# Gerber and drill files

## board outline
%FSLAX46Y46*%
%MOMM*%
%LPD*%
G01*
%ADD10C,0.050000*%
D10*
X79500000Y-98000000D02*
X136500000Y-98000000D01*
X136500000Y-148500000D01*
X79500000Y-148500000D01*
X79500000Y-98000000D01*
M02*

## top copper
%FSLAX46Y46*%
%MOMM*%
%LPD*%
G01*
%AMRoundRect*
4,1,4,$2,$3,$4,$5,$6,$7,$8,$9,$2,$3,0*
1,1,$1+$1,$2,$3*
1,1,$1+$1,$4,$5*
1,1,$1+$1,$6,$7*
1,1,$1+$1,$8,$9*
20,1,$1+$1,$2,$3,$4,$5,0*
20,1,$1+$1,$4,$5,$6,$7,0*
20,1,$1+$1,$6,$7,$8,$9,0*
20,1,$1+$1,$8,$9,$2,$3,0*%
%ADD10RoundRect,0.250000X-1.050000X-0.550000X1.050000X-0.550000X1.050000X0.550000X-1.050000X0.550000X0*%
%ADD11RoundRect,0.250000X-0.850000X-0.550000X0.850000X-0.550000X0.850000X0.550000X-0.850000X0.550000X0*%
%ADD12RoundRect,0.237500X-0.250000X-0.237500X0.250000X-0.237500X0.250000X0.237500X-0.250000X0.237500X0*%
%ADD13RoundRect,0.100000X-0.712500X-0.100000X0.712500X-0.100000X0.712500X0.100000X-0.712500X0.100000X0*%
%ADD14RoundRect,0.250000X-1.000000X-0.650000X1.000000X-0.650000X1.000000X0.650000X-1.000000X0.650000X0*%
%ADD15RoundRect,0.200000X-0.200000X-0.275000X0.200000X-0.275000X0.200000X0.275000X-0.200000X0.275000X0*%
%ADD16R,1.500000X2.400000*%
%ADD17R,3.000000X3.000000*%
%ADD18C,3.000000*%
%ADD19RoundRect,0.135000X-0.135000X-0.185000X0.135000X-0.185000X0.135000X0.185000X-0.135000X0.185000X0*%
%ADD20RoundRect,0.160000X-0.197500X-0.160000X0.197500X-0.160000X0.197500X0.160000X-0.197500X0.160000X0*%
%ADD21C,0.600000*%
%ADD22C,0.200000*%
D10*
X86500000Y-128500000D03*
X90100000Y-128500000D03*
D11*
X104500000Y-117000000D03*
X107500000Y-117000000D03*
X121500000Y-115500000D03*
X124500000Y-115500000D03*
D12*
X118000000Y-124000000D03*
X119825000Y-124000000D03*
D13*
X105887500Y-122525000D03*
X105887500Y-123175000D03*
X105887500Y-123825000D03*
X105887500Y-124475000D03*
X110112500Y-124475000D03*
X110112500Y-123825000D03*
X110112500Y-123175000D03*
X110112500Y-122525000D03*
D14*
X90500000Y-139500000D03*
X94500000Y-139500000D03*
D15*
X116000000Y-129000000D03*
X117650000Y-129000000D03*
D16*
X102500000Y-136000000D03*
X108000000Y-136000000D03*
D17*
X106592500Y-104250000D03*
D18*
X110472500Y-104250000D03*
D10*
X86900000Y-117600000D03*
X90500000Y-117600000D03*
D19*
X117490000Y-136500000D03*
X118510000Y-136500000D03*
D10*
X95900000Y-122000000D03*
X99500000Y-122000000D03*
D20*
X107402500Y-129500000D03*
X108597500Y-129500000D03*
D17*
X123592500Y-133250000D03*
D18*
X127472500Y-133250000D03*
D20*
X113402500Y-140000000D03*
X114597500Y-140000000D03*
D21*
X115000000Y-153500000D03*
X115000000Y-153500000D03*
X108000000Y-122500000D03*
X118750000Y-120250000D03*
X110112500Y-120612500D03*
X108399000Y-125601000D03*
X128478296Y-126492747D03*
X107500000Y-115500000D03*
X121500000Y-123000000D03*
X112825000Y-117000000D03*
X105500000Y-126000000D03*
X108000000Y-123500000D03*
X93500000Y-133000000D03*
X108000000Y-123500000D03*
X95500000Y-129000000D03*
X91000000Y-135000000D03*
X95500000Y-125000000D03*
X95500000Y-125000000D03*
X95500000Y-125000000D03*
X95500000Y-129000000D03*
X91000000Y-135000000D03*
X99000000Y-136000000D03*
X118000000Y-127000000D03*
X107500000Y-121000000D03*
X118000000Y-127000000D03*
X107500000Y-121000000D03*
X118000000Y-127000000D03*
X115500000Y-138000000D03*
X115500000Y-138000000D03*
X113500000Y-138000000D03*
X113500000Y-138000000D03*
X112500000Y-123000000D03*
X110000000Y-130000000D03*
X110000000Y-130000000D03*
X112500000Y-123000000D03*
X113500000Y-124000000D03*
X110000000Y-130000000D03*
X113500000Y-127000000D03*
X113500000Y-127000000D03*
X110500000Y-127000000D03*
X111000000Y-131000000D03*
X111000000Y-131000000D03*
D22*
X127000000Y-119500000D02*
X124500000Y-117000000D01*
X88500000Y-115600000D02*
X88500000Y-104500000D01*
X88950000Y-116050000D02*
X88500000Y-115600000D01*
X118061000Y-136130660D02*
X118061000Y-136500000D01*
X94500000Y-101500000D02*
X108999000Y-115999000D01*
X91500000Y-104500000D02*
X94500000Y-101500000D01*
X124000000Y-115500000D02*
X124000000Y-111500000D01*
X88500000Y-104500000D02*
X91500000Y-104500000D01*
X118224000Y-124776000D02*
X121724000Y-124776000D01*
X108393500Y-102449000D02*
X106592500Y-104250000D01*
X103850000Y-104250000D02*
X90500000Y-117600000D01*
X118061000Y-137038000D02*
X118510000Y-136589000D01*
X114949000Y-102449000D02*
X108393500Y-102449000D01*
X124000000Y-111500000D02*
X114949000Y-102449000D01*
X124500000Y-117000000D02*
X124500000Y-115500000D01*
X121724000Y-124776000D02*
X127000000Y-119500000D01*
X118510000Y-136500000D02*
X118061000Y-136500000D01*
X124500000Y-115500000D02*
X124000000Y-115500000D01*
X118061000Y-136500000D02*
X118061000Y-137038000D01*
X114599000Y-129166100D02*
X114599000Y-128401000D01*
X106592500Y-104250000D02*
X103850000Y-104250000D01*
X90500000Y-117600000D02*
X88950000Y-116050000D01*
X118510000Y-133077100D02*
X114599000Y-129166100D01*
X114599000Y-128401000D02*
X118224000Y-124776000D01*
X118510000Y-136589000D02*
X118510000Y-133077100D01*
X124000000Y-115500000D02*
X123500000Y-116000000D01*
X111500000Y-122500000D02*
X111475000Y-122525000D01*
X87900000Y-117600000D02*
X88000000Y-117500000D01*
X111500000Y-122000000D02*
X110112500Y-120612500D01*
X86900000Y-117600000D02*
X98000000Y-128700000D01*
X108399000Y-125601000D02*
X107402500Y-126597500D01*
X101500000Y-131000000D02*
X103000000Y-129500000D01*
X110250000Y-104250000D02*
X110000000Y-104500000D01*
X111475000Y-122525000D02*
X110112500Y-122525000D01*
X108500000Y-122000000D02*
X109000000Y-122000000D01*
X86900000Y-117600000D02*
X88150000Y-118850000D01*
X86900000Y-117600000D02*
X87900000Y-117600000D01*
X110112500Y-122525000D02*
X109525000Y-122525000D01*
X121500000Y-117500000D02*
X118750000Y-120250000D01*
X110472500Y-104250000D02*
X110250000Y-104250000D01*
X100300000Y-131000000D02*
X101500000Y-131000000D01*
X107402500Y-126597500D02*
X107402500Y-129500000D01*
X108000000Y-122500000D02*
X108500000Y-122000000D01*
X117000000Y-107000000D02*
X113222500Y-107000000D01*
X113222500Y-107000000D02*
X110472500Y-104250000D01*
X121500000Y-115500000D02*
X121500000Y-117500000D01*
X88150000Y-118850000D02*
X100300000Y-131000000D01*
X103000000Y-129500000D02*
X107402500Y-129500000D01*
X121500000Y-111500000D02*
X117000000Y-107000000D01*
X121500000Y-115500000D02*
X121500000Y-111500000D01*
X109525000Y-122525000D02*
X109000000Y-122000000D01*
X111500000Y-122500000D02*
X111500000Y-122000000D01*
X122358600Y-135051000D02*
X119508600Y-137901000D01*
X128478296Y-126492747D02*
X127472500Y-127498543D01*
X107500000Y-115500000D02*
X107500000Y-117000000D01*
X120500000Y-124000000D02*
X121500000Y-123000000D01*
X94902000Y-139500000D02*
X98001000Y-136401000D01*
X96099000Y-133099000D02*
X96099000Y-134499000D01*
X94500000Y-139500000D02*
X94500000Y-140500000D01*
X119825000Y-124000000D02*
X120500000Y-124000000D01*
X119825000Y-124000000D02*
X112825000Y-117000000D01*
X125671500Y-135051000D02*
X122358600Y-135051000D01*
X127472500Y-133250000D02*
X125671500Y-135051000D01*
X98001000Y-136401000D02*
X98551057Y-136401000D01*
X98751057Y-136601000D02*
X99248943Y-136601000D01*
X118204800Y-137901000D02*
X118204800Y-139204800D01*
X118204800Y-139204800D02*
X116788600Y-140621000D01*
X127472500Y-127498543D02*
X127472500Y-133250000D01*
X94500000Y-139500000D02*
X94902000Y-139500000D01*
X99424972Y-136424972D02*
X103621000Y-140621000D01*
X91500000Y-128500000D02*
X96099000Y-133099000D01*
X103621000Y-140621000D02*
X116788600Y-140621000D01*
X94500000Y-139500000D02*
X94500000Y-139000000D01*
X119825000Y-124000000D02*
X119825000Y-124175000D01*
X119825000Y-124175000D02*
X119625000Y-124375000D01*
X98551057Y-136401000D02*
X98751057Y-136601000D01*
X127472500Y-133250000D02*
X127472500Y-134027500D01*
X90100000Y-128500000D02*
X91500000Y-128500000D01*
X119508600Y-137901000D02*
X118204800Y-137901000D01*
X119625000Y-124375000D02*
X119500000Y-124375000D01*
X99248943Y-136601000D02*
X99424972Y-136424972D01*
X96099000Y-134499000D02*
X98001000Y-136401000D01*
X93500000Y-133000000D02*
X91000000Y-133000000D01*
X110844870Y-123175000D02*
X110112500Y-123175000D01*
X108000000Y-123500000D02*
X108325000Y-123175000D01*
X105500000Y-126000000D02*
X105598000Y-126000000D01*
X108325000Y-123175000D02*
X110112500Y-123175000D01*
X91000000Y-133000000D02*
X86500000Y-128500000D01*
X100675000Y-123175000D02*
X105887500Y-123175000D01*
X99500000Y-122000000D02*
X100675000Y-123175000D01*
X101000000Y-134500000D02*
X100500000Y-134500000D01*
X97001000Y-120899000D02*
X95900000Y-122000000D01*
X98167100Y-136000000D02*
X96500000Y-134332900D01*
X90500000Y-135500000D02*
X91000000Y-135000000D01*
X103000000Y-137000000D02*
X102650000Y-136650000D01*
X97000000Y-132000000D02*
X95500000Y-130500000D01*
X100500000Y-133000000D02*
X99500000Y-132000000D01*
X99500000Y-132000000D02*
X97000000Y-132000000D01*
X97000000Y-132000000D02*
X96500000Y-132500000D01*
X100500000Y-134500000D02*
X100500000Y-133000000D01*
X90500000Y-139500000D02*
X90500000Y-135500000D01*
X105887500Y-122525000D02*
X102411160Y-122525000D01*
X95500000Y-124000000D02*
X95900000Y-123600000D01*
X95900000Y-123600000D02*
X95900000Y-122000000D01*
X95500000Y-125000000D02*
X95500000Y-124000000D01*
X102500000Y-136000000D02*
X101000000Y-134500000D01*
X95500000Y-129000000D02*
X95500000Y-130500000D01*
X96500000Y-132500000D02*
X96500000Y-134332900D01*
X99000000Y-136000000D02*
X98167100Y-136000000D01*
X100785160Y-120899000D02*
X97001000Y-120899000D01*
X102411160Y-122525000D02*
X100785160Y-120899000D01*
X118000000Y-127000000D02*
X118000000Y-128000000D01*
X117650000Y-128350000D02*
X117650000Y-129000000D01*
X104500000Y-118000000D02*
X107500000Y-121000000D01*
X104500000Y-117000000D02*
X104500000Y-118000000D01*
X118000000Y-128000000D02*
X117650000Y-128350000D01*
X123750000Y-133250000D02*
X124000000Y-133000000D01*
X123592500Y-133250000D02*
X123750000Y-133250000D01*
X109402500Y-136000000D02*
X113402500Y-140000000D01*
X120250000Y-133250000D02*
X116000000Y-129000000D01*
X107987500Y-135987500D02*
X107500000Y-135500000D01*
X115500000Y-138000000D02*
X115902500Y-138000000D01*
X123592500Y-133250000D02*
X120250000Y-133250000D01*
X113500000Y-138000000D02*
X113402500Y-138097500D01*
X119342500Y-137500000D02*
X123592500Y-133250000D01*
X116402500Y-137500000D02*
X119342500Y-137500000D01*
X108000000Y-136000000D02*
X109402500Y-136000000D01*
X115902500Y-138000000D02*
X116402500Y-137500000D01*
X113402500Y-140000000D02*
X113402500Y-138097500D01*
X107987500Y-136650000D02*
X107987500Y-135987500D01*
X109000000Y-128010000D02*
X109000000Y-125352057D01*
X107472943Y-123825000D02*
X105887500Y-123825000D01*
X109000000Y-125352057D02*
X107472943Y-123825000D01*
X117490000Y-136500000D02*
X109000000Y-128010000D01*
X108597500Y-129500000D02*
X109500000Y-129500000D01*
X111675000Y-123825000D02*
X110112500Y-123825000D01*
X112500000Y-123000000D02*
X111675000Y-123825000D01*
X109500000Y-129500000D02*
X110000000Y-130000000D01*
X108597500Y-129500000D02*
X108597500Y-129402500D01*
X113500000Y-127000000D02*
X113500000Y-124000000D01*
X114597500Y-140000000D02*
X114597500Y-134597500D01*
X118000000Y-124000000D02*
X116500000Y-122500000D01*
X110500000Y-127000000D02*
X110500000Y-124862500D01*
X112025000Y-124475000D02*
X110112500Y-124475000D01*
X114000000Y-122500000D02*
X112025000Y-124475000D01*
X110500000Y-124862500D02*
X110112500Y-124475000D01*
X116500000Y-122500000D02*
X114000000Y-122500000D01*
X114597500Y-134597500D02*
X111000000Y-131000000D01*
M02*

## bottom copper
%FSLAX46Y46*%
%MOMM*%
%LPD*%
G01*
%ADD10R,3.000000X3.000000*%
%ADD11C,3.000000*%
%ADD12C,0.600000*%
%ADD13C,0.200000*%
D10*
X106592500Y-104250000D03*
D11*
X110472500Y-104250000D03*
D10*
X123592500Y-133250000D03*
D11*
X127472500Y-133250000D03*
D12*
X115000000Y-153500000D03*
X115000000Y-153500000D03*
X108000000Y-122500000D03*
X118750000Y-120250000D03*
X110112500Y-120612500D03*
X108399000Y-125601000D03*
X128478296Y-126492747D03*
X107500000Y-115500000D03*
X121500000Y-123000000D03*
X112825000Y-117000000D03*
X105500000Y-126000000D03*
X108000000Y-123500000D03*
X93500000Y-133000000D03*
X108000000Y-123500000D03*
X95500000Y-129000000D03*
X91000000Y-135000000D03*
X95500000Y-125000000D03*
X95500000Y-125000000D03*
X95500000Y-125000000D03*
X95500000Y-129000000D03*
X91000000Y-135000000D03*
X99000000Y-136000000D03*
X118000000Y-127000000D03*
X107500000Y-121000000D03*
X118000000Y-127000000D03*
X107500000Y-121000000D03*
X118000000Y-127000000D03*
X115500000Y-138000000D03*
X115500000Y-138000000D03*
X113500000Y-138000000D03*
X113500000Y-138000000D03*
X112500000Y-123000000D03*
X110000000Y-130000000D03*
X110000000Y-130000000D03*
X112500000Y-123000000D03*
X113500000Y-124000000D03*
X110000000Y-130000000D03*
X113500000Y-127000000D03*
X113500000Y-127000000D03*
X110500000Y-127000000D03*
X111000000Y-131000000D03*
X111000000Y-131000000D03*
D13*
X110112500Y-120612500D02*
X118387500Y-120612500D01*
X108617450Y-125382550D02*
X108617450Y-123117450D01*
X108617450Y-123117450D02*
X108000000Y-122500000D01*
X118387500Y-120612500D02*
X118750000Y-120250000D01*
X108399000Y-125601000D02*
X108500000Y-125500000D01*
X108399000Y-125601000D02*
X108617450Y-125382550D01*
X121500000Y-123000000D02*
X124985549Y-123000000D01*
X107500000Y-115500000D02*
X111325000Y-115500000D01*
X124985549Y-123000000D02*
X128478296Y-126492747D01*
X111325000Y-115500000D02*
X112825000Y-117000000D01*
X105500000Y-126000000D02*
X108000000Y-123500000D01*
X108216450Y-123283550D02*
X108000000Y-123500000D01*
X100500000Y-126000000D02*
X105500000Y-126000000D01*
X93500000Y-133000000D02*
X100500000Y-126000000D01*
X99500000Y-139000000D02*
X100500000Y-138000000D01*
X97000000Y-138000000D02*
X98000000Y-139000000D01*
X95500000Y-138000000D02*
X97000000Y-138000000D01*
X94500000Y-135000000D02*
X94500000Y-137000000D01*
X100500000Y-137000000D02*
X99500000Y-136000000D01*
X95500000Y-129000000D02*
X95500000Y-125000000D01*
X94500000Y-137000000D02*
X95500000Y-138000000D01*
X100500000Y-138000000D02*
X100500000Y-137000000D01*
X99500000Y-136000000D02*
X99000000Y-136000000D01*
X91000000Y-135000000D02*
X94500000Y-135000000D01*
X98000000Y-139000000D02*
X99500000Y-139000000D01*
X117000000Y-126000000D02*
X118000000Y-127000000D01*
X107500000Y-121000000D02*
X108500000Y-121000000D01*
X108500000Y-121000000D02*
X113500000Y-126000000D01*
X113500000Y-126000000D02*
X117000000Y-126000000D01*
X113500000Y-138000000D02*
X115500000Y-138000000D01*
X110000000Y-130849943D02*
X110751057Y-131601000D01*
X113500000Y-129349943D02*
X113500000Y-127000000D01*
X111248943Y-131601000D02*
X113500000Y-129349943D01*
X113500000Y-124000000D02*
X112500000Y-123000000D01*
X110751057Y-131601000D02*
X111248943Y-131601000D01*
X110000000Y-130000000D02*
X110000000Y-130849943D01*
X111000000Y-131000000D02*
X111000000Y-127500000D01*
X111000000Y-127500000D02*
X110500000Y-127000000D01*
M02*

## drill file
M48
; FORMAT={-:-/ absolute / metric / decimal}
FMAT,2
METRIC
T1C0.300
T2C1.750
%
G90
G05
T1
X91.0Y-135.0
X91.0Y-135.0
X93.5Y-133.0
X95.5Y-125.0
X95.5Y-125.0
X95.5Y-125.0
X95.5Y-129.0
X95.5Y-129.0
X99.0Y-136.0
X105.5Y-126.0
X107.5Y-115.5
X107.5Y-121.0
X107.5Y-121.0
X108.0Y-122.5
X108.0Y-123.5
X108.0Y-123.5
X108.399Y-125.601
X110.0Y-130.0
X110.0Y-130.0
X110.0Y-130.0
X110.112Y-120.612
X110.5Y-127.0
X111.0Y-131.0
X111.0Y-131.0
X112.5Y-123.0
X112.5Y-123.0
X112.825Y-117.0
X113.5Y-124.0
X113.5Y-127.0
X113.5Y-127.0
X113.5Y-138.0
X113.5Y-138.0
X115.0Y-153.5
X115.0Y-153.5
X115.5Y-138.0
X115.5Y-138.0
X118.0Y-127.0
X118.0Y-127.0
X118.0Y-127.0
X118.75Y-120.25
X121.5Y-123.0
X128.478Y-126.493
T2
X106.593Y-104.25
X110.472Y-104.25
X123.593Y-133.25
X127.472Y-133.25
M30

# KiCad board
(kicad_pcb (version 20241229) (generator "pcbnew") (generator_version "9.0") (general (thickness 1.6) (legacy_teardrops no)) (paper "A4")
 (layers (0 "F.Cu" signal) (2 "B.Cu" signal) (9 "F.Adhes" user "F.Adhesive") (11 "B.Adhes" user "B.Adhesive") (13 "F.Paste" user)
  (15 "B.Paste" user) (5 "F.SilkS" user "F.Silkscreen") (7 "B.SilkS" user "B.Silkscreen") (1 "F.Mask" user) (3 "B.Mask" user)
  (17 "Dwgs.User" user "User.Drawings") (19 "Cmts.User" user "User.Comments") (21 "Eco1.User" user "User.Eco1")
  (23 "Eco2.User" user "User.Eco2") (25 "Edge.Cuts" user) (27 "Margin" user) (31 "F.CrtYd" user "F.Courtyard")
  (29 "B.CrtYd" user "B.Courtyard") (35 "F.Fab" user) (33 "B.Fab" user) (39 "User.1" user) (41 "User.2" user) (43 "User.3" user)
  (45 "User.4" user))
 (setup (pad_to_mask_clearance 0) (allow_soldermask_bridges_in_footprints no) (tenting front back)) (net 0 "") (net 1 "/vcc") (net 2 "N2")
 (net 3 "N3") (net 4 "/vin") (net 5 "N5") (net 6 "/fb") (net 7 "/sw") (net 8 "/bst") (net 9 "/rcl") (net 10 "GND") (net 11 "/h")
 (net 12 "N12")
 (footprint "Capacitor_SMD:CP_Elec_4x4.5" (layer "F.Cu") (at 88.3 128.5)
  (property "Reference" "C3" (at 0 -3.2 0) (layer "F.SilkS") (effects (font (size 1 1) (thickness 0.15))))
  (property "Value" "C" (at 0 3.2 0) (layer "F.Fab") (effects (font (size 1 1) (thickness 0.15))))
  (pad "1" smd roundrect (at -1.8 0) (size 2.6 1.6) (layers "F.Cu" "F.Mask" "F.Paste") (roundrect_rratio 0.15625) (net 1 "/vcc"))
  (pad "2" smd roundrect (at 1.8 0) (size 2.6 1.6) (layers "F.Cu" "F.Mask" "F.Paste") (roundrect_rratio 0.15625) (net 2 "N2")))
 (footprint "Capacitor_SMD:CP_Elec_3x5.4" (layer "F.Cu") (at 106 117)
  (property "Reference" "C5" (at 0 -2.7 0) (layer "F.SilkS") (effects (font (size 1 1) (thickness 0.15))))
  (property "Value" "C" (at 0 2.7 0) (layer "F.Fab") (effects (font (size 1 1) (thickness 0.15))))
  (pad "1" smd roundrect (at -1.5 0) (size 2.2 1.6) (layers "F.Cu" "F.Mask" "F.Paste") (roundrect_rratio 0.15625) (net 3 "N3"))
  (pad "2" smd roundrect (at 1.5 0) (size 2.2 1.6) (layers "F.Cu" "F.Mask" "F.Paste") (roundrect_rratio 0.15625) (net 2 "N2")))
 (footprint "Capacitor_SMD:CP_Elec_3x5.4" (layer "F.Cu") (at 123 115.5)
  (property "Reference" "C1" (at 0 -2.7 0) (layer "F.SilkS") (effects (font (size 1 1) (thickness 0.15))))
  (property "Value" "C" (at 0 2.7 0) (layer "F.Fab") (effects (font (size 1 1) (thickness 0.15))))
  (pad "1" smd roundrect (at -1.5 0) (size 2.2 1.6) (layers "F.Cu" "F.Mask" "F.Paste") (roundrect_rratio 0.15625) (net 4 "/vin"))
  (pad "2" smd roundrect (at 1.5 0) (size 2.2 1.6) (layers "F.Cu" "F.Mask" "F.Paste") (roundrect_rratio 0.15625) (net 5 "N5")))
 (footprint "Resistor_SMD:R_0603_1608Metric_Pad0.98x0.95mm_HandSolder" (layer "F.Cu") (at 118.9125 124)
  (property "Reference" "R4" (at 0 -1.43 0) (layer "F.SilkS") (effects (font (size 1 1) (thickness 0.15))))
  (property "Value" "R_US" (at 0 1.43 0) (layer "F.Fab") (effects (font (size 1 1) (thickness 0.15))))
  (pad "1" smd roundrect (at -0.9125 0) (size 0.975 0.95) (layers "F.Cu" "F.Mask" "F.Paste") (roundrect_rratio 0.25) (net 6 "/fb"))
  (pad "2" smd roundrect (at 0.9125 0) (size 0.975 0.95) (layers "F.Cu" "F.Mask" "F.Paste") (roundrect_rratio 0.25) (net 2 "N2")))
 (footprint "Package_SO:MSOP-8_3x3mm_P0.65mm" (layer "F.Cu") (at 108 123.5)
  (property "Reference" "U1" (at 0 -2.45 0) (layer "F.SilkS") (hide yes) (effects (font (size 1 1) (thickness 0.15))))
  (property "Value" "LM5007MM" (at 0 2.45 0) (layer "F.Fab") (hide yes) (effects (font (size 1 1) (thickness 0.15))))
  (pad "1" smd roundrect (at -2.1125 -0.975) (size 1.625 0.4) (layers "F.Cu" "F.Mask" "F.Paste") (roundrect_rratio 0.25) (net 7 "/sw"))
  (pad "2" smd roundrect (at -2.1125 -0.325) (size 1.625 0.4) (layers "F.Cu" "F.Mask" "F.Paste") (roundrect_rratio 0.25) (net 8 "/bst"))
  (pad "3" smd roundrect (at -2.1125 0.325) (size 1.625 0.4) (layers "F.Cu" "F.Mask" "F.Paste") (roundrect_rratio 0.25) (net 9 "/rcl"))
  (pad "4" smd roundrect (at -2.1125 0.975) (size 1.625 0.4) (layers "F.Cu" "F.Mask" "F.Paste") (roundrect_rratio 0.25) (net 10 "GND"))
  (pad "5" smd roundrect (at 2.1125 0.975) (size 1.625 0.4) (layers "F.Cu" "F.Mask" "F.Paste") (roundrect_rratio 0.25) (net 6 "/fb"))
  (pad "6" smd roundrect (at 2.1125 0.325) (size 1.625 0.4) (layers "F.Cu" "F.Mask" "F.Paste") (roundrect_rratio 0.25) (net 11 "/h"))
  (pad "7" smd roundrect (at 2.1125 -0.325) (size 1.625 0.4) (layers "F.Cu" "F.Mask" "F.Paste") (roundrect_rratio 0.25) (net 1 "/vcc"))
  (pad "8" smd roundrect (at 2.1125 -0.975) (size 1.625 0.4) (layers "F.Cu" "F.Mask" "F.Paste") (roundrect_rratio 0.25) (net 4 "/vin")))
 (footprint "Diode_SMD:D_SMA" (layer "F.Cu") (at 92.5 139.5)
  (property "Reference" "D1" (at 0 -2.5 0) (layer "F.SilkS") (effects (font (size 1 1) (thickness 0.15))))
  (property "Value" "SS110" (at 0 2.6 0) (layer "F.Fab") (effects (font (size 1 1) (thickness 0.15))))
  (pad "1" smd roundrect (at -2 0) (size 2.5 1.8) (layers "F.Cu" "F.Mask" "F.Paste") (roundrect_rratio 0.1388888889) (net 7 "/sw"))
  (pad "2" smd roundrect (at 2 0) (size 2.5 1.8) (layers "F.Cu" "F.Mask" "F.Paste") (roundrect_rratio 0.1388888889) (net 2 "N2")))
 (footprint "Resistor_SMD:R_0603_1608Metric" (layer "F.Cu") (at 116.825 129)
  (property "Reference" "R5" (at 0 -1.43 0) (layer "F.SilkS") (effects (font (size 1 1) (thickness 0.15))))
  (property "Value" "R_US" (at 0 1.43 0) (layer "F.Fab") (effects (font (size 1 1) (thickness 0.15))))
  (pad "1" smd roundrect (at -0.825 0) (size 0.8 0.95) (layers "F.Cu" "F.Mask" "F.Paste") (roundrect_rratio 0.25) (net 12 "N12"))
  (pad "2" smd roundrect (at 0.825 0) (size 0.8 0.95) (layers "F.Cu" "F.Mask" "F.Paste") (roundrect_rratio 0.25) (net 3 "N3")))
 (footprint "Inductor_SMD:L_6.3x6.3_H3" (layer "F.Cu") (at 105.25 136)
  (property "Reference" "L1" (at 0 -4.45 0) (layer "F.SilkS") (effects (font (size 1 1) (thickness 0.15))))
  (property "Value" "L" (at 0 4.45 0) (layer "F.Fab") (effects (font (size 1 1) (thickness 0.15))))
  (pad "1" smd rect (at -2.75 0) (size 1.5 2.4) (layers "F.Cu" "F.Mask" "F.Paste") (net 7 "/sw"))
  (pad "2" smd rect (at 2.75 0) (size 1.5 2.4) (layers "F.Cu" "F.Mask" "F.Paste") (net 12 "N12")))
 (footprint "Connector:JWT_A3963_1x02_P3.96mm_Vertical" (layer "F.Cu") (at 106.5925 104.25)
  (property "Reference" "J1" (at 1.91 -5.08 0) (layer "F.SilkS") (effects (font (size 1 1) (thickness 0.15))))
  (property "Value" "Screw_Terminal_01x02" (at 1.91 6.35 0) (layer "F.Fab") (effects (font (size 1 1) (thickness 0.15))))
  (pad "1" thru_hole rect (at 0 0) (size 3 3) (drill 1.75) (layers "*.Cu" "*.Mask") (remove_unused_layers no) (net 5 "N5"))
  (pad "2" thru_hole circle (at 3.88 0) (size 3 3) (drill 1.75) (layers "*.Cu" "*.Mask") (remove_unused_layers no) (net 4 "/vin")))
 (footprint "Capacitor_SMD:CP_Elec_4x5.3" (layer "F.Cu") (at 88.7 117.6)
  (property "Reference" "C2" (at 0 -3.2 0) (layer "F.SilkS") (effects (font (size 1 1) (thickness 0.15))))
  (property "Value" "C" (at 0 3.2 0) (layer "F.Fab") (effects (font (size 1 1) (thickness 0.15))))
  (pad "1" smd roundrect (at -1.8 0) (size 2.6 1.6) (layers "F.Cu" "F.Mask" "F.Paste") (roundrect_rratio 0.15625) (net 4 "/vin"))
  (pad "2" smd roundrect (at 1.8 0) (size 2.6 1.6) (layers "F.Cu" "F.Mask" "F.Paste") (roundrect_rratio 0.15625) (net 5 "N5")))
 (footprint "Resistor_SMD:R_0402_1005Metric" (layer "F.Cu") (at 118 136.5)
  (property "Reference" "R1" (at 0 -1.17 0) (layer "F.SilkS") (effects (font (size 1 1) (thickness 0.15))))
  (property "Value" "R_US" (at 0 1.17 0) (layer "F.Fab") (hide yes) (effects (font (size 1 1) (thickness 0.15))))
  (pad "1" smd roundrect (at -0.51 0) (size 0.54 0.64) (layers "F.Cu" "F.Mask" "F.Paste") (roundrect_rratio 0.25) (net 9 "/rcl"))
  (pad "2" smd roundrect (at 0.51 0) (size 0.54 0.64) (layers "F.Cu" "F.Mask" "F.Paste") (roundrect_rratio 0.25) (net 5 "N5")))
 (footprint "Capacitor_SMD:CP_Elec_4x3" (layer "F.Cu") (at 97.7 122)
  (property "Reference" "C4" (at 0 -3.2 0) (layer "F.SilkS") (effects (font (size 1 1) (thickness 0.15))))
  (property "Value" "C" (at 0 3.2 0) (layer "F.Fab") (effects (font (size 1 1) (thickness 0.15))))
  (pad "1" smd roundrect (at -1.8 0) (size 2.6 1.6) (layers "F.Cu" "F.Mask" "F.Paste") (roundrect_rratio 0.15625) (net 7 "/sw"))
  (pad "2" smd roundrect (at 1.8 0) (size 2.6 1.6) (layers "F.Cu" "F.Mask" "F.Paste") (roundrect_rratio 0.15625) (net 8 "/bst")))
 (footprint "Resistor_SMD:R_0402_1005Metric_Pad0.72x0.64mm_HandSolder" (layer "F.Cu") (at 108 129.5)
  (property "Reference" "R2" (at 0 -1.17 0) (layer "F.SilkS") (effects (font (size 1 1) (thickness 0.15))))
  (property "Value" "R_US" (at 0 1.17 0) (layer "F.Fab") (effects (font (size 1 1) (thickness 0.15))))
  (pad "1" smd roundrect (at -0.5975 0) (size 0.715 0.64) (layers "F.Cu" "F.Mask" "F.Paste") (roundrect_rratio 0.25) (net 4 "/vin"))
  (pad "2" smd roundrect (at 0.5975 0) (size 0.715 0.64) (layers "F.Cu" "F.Mask" "F.Paste") (roundrect_rratio 0.25) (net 11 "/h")))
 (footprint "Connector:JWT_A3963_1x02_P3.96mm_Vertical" (layer "F.Cu") (at 123.5925 133.25)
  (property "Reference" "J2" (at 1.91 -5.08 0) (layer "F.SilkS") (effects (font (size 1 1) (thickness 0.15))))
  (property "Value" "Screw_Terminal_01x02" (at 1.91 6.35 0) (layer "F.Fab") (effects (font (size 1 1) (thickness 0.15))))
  (pad "1" thru_hole rect (at 0 0) (size 3 3) (drill 1.75) (layers "*.Cu" "*.Mask") (remove_unused_layers no) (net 12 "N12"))
  (pad "2" thru_hole circle (at 3.88 0) (size 3 3) (drill 1.75) (layers "*.Cu" "*.Mask") (remove_unused_layers no) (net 2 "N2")))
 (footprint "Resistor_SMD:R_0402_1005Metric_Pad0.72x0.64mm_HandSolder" (layer "F.Cu") (at 114 140)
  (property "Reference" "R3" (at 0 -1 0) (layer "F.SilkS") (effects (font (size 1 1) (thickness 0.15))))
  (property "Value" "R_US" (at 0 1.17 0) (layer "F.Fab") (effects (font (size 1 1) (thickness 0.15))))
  (pad "1" smd roundrect (at -0.5975 0) (size 0.715 0.64) (layers "F.Cu" "F.Mask" "F.Paste") (roundrect_rratio 0.25) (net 12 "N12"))
  (pad "2" smd roundrect (at 0.5975 0) (size 0.715 0.64) (layers "F.Cu" "F.Mask" "F.Paste") (roundrect_rratio 0.25) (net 6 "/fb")))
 (gr_rect (start 79.5 98) (end 136.5 148.5) (stroke (width 0.05) (type default)) (fill no) (layer "Edge.Cuts"))
 (via (at 115 153.5) (size 0.6) (drill 0.3) (layers "F.Cu" "B.Cu") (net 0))
 (via (at 115 153.5) (size 0.6) (drill 0.3) (layers "F.Cu" "B.Cu") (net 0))
 (segment (start 127 119.5) (end 124.5 117) (width 0.2) (layer "F.Cu") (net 5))
 (segment (start 88.5 115.6) (end 88.5 104.5) (width 0.2) (layer "F.Cu") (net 5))
 (segment (start 88.95 116.05) (end 88.5 115.6) (width 0.2) (layer "F.Cu") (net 5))
 (segment (start 118.061 136.13066) (end 118.061 136.5) (width 0.2) (layer "F.Cu") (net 5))
 (segment (start 94.5 101.5) (end 108.999 115.999) (width 0.2) (layer "F.Cu") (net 5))
 (segment (start 91.5 104.5) (end 94.5 101.5) (width 0.2) (layer "F.Cu") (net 5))
 (segment (start 124 115.5) (end 124 111.5) (width 0.2) (layer "F.Cu") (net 5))
 (segment (start 88.5 104.5) (end 91.5 104.5) (width 0.2) (layer "F.Cu") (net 5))
 (segment (start 118.224 124.776) (end 121.724 124.776) (width 0.2) (layer "F.Cu") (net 5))
 (segment (start 108.3935 102.449) (end 106.5925 104.25) (width 0.2) (layer "F.Cu") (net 5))
 (segment (start 103.85 104.25) (end 90.5 117.6) (width 0.2) (layer "F.Cu") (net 5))
 (segment (start 118.061 137.038) (end 118.51 136.589) (width 0.2) (layer "F.Cu") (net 5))
 (segment (start 114.949 102.449) (end 108.3935 102.449) (width 0.2) (layer "F.Cu") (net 5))
 (segment (start 124 111.5) (end 114.949 102.449) (width 0.2) (layer "F.Cu") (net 5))
 (segment (start 124.5 117) (end 124.5 115.5) (width 0.2) (layer "F.Cu") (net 5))
 (segment (start 121.724 124.776) (end 127 119.5) (width 0.2) (layer "F.Cu") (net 5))
 (segment (start 118.51 136.5) (end 118.061 136.5) (width 0.2) (layer "F.Cu") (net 5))
 (segment (start 124.5 115.5) (end 124 115.5) (width 0.2) (layer "F.Cu") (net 5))
 (segment (start 118.061 136.5) (end 118.061 137.038) (width 0.2) (layer "F.Cu") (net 5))
 (segment (start 114.599 129.1661) (end 114.599 128.401) (width 0.2) (layer "F.Cu") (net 5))
 (segment (start 106.5925 104.25) (end 103.85 104.25) (width 0.2) (layer "F.Cu") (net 5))
 (segment (start 90.5 117.6) (end 88.95 116.05) (width 0.2) (layer "F.Cu") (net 5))
 (segment (start 118.51 133.0771) (end 114.599 129.1661) (width 0.2) (layer "F.Cu") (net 5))
 (segment (start 114.599 128.401) (end 118.224 124.776) (width 0.2) (layer "F.Cu") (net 5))
 (segment (start 118.51 136.589) (end 118.51 133.0771) (width 0.2) (layer "F.Cu") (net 5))
 (segment (start 124 115.5) (end 123.5 116) (width 0.2) (layer "F.Cu") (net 5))
 (segment (start 111.5 122.5) (end 111.475 122.525) (width 0.2) (layer "F.Cu") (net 4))
 (segment (start 87.9 117.6) (end 88 117.5) (width 0.2) (layer "F.Cu") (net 4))
 (segment (start 111.5 122) (end 110.1125 120.6125) (width 0.2) (layer "F.Cu") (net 4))
 (segment (start 86.9 117.6) (end 98 128.7) (width 0.2) (layer "F.Cu") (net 4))
 (segment (start 108.399 125.601) (end 107.4025 126.5975) (width 0.2) (layer "F.Cu") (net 4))
 (segment (start 101.5 131) (end 103 129.5) (width 0.2) (layer "F.Cu") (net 4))
 (segment (start 110.25 104.25) (end 110 104.5) (width 0.2) (layer "F.Cu") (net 4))
 (segment (start 111.475 122.525) (end 110.1125 122.525) (width 0.2) (layer "F.Cu") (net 4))
 (segment (start 108.5 122) (end 109 122) (width 0.2) (layer "F.Cu") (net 4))
 (segment (start 86.9 117.6) (end 88.15 118.85) (width 0.2) (layer "F.Cu") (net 4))
 (segment (start 86.9 117.6) (end 87.9 117.6) (width 0.2) (layer "F.Cu") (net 4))
 (segment (start 110.1125 122.525) (end 109.525 122.525) (width 0.2) (layer "F.Cu") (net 4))
 (segment (start 121.5 117.5) (end 118.75 120.25) (width 0.2) (layer "F.Cu") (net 4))
 (segment (start 110.4725 104.25) (end 110.25 104.25) (width 0.2) (layer "F.Cu") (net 4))
 (segment (start 100.3 131) (end 101.5 131) (width 0.2) (layer "F.Cu") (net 4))
 (segment (start 107.4025 126.5975) (end 107.4025 129.5) (width 0.2) (layer "F.Cu") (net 4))
 (segment (start 108 122.5) (end 108.5 122) (width 0.2) (layer "F.Cu") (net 4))
 (segment (start 117 107) (end 113.2225 107) (width 0.2) (layer "F.Cu") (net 4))
 (segment (start 113.2225 107) (end 110.4725 104.25) (width 0.2) (layer "F.Cu") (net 4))
 (segment (start 121.5 115.5) (end 121.5 117.5) (width 0.2) (layer "F.Cu") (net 4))
 (segment (start 88.15 118.85) (end 100.3 131) (width 0.2) (layer "F.Cu") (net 4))
 (segment (start 103 129.5) (end 107.4025 129.5) (width 0.2) (layer "F.Cu") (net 4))
 (segment (start 121.5 111.5) (end 117 107) (width 0.2) (layer "F.Cu") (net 4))
 (segment (start 121.5 115.5) (end 121.5 111.5) (width 0.2) (layer "F.Cu") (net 4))
 (segment (start 109.525 122.525) (end 109 122) (width 0.2) (layer "F.Cu") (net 4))
 (segment (start 111.5 122.5) (end 111.5 122) (width 0.2) (layer "F.Cu") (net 4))
 (via (at 108 122.5) (size 0.6) (drill 0.3) (layers "F.Cu" "B.Cu") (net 4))
 (via (at 118.75 120.25) (size 0.6) (drill 0.3) (layers "F.Cu" "B.Cu") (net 4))
 (via (at 110.1125 120.6125) (size 0.6) (drill 0.3) (layers "F.Cu" "B.Cu") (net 4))
 (via (at 108.399 125.601) (size 0.6) (drill 0.3) (layers "F.Cu" "B.Cu") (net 4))
 (segment (start 110.1125 120.6125) (end 118.3875 120.6125) (width 0.2) (layer "B.Cu") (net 4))
 (segment (start 108.61745 125.38255) (end 108.61745 123.11745) (width 0.2) (layer "B.Cu") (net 4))
 (segment (start 108.61745 123.11745) (end 108 122.5) (width 0.2) (layer "B.Cu") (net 4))
 (segment (start 118.3875 120.6125) (end 118.75 120.25) (width 0.2) (layer "B.Cu") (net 4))
 (segment (start 108.399 125.601) (end 108.5 125.5) (width 0.2) (layer "B.Cu") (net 4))
 (segment (start 108.399 125.601) (end 108.61745 125.38255) (width 0.2) (layer "B.Cu") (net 4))
 (segment (start 122.3586 135.051) (end 119.5086 137.901) (width 0.2) (layer "F.Cu") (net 2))
 (segment (start 128.478296 126.492747) (end 127.4725 127.498543) (width 0.2) (layer "F.Cu") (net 2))
 (segment (start 107.5 115.5) (end 107.5 117) (width 0.2) (layer "F.Cu") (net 2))
 (segment (start 120.5 124) (end 121.5 123) (width 0.2) (layer "F.Cu") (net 2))
 (segment (start 94.902 139.5) (end 98.001 136.401) (width 0.2) (layer "F.Cu") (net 2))
 (segment (start 96.099 133.099) (end 96.099 134.499) (width 0.2) (layer "F.Cu") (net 2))
 (segment (start 94.5 139.5) (end 94.5 140.5) (width 0.2) (layer "F.Cu") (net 2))
 (segment (start 119.825 124) (end 120.5 124) (width 0.2) (layer "F.Cu") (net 2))
 (segment (start 119.825 124) (end 112.825 117) (width 0.2) (layer "F.Cu") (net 2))
 (segment (start 125.6715 135.051) (end 122.3586 135.051) (width 0.2) (layer "F.Cu") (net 2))
 (segment (start 127.4725 133.25) (end 125.6715 135.051) (width 0.2) (layer "F.Cu") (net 2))
 (segment (start 98.001 136.401) (end 98.551057 136.401) (width 0.2) (layer "F.Cu") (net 2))
 (segment (start 98.751057 136.601) (end 99.248943 136.601) (width 0.2) (layer "F.Cu") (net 2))
 (segment (start 118.2048 137.901) (end 118.2048 139.2048) (width 0.2) (layer "F.Cu") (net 2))
 (segment (start 118.2048 139.2048) (end 116.7886 140.621) (width 0.2) (layer "F.Cu") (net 2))
 (segment (start 127.4725 127.498543) (end 127.4725 133.25) (width 0.2) (layer "F.Cu") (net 2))
 (segment (start 94.5 139.5) (end 94.902 139.5) (width 0.2) (layer "F.Cu") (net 2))
 (segment (start 99.424972 136.424972) (end 103.621 140.621) (width 0.2) (layer "F.Cu") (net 2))
 (segment (start 91.5 128.5) (end 96.099 133.099) (width 0.2) (layer "F.Cu") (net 2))
 (segment (start 103.621 140.621) (end 116.7886 140.621) (width 0.2) (layer "F.Cu") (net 2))
 (segment (start 94.5 139.5) (end 94.5 139) (width 0.2) (layer "F.Cu") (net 2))
 (segment (start 119.825 124) (end 119.825 124.175) (width 0.2) (layer "F.Cu") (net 2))
 (segment (start 119.825 124.175) (end 119.625 124.375) (width 0.2) (layer "F.Cu") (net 2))
 (segment (start 98.551057 136.401) (end 98.751057 136.601) (width 0.2) (layer "F.Cu") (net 2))
 (segment (start 127.4725 133.25) (end 127.4725 134.0275) (width 0.2) (layer "F.Cu") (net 2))
 (segment (start 90.1 128.5) (end 91.5 128.5) (width 0.2) (layer "F.Cu") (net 2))
 (segment (start 119.5086 137.901) (end 118.2048 137.901) (width 0.2) (layer "F.Cu") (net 2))
 (segment (start 119.625 124.375) (end 119.5 124.375) (width 0.2) (layer "F.Cu") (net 2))
 (segment (start 99.248943 136.601) (end 99.424972 136.424972) (width 0.2) (layer "F.Cu") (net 2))
 (segment (start 96.099 134.499) (end 98.001 136.401) (width 0.2) (layer "F.Cu") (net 2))
 (via (at 128.478296 126.492747) (size 0.6) (drill 0.3) (layers "F.Cu" "B.Cu") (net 2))
 (via (at 107.5 115.5) (size 0.6) (drill 0.3) (layers "F.Cu" "B.Cu") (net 2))
 (via (at 121.5 123) (size 0.6) (drill 0.3) (layers "F.Cu" "B.Cu") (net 2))
 (via (at 112.825 117) (size 0.6) (drill 0.3) (layers "F.Cu" "B.Cu") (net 2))
 (segment (start 121.5 123) (end 124.985549 123) (width 0.2) (layer "B.Cu") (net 2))
 (segment (start 107.5 115.5) (end 111.325 115.5) (width 0.2) (layer "B.Cu") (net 2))
 (segment (start 124.985549 123) (end 128.478296 126.492747) (width 0.2) (layer "B.Cu") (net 2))
 (segment (start 111.325 115.5) (end 112.825 117) (width 0.2) (layer "B.Cu") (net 2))
 (segment (start 93.5 133) (end 91 133) (width 0.2) (layer "F.Cu") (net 1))
 (segment (start 110.84487 123.175) (end 110.1125 123.175) (width 0.2) (layer "F.Cu") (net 1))
 (segment (start 108 123.5) (end 108.325 123.175) (width 0.2) (layer "F.Cu") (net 1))
 (segment (start 105.5 126) (end 105.598 126) (width 0.2) (layer "F.Cu") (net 1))
 (segment (start 108.325 123.175) (end 110.1125 123.175) (width 0.2) (layer "F.Cu") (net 1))
 (segment (start 91 133) (end 86.5 128.5) (width 0.2) (layer "F.Cu") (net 1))
 (via (at 105.5 126) (size 0.6) (drill 0.3) (layers "F.Cu" "B.Cu") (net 1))
 (via (at 108 123.5) (size 0.6) (drill 0.3) (layers "F.Cu" "B.Cu") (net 1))
 (via (at 93.5 133) (size 0.6) (drill 0.3) (layers "F.Cu" "B.Cu") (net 1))
 (via (at 108 123.5) (size 0.6) (drill 0.3) (layers "F.Cu" "B.Cu") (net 1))
 (segment (start 105.5 126) (end 108 123.5) (width 0.2) (layer "B.Cu") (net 1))
 (segment (start 108.21645 123.28355) (end 108 123.5) (width 0.2) (layer "B.Cu") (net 1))
 (segment (start 100.5 126) (end 105.5 126) (width 0.2) (layer "B.Cu") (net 1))
 (segment (start 93.5 133) (end 100.5 126) (width 0.2) (layer "B.Cu") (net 1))
 (segment (start 100.675 123.175) (end 105.8875 123.175) (width 0.2) (layer "F.Cu") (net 8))
 (segment (start 99.5 122) (end 100.675 123.175) (width 0.2) (layer "F.Cu") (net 8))
 (segment (start 101 134.5) (end 100.5 134.5) (width 0.2) (layer "F.Cu") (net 7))
 (segment (start 97.001 120.899) (end 95.9 122) (width 0.2) (layer "F.Cu") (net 7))
 (segment (start 98.1671 136) (end 96.5 134.3329) (width 0.2) (layer "F.Cu") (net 7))
 (segment (start 90.5 135.5) (end 91 135) (width 0.2) (layer "F.Cu") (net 7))
 (segment (start 103 137) (end 102.65 136.65) (width 0.2) (layer "F.Cu") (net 7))
 (segment (start 97 132) (end 95.5 130.5) (width 0.2) (layer "F.Cu") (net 7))
 (segment (start 100.5 133) (end 99.5 132) (width 0.2) (layer "F.Cu") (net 7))
 (segment (start 99.5 132) (end 97 132) (width 0.2) (layer "F.Cu") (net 7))
 (segment (start 97 132) (end 96.5 132.5) (width 0.2) (layer "F.Cu") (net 7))
 (segment (start 100.5 134.5) (end 100.5 133) (width 0.2) (layer "F.Cu") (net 7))
 (segment (start 90.5 139.5) (end 90.5 135.5) (width 0.2) (layer "F.Cu") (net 7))
 (segment (start 105.8875 122.525) (end 102.41116 122.525) (width 0.2) (layer "F.Cu") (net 7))
 (segment (start 95.5 124) (end 95.9 123.6) (width 0.2) (layer "F.Cu") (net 7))
 (segment (start 95.9 123.6) (end 95.9 122) (width 0.2) (layer "F.Cu") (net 7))
 (segment (start 95.5 125) (end 95.5 124) (width 0.2) (layer "F.Cu") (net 7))
 (segment (start 102.5 136) (end 101 134.5) (width 0.2) (layer "F.Cu") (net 7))
 (segment (start 95.5 129) (end 95.5 130.5) (width 0.2) (layer "F.Cu") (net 7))
 (segment (start 96.5 132.5) (end 96.5 134.3329) (width 0.2) (layer "F.Cu") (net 7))
 (segment (start 99 136) (end 98.1671 136) (width 0.2) (layer "F.Cu") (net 7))
 (segment (start 100.78516 120.899) (end 97.001 120.899) (width 0.2) (layer "F.Cu") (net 7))
 (segment (start 102.41116 122.525) (end 100.78516 120.899) (width 0.2) (layer "F.Cu") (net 7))
 (via (at 95.5 129) (size 0.6) (drill 0.3) (layers "F.Cu" "B.Cu") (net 7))
 (via (at 91 135) (size 0.6) (drill 0.3) (layers "F.Cu" "B.Cu") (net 7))
 (via (at 95.5 125) (size 0.6) (drill 0.3) (layers "F.Cu" "B.Cu") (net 7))
 (via (at 95.5 125) (size 0.6) (drill 0.3) (layers "F.Cu" "B.Cu") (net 7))
 (via (at 95.5 125) (size 0.6) (drill 0.3) (layers "F.Cu" "B.Cu") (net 7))
 (via (at 95.5 129) (size 0.6) (drill 0.3) (layers "F.Cu" "B.Cu") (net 7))
 (via (at 91 135) (size 0.6) (drill 0.3) (layers "F.Cu" "B.Cu") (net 7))
 (via (at 99 136) (size 0.6) (drill 0.3) (layers "F.Cu" "B.Cu") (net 7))
 (segment (start 99.5 139) (end 100.5 138) (width 0.2) (layer "B.Cu") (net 7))
 (segment (start 97 138) (end 98 139) (width 0.2) (layer "B.Cu") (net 7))
 (segment (start 95.5 138) (end 97 138) (width 0.2) (layer "B.Cu") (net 7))
 (segment (start 94.5 135) (end 94.5 137) (width 0.2) (layer "B.Cu") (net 7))
 (segment (start 100.5 137) (end 99.5 136) (width 0.2) (layer "B.Cu") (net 7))
 (segment (start 95.5 129) (end 95.5 125) (width 0.2) (layer "B.Cu") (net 7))
 (segment (start 94.5 137) (end 95.5 138) (width 0.2) (layer "B.Cu") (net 7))
 (segment (start 100.5 138) (end 100.5 137) (width 0.2) (layer "B.Cu") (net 7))
 (segment (start 99.5 136) (end 99 136) (width 0.2) (layer "B.Cu") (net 7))
 (segment (start 91 135) (end 94.5 135) (width 0.2) (layer "B.Cu") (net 7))
 (segment (start 98 139) (end 99.5 139) (width 0.2) (layer "B.Cu") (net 7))
 (segment (start 118 127) (end 118 128) (width 0.2) (layer "F.Cu") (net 3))
 (segment (start 117.65 128.35) (end 117.65 129) (width 0.2) (layer "F.Cu") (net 3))
 (segment (start 104.5 118) (end 107.5 121) (width 0.2) (layer "F.Cu") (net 3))
 (segment (start 104.5 117) (end 104.5 118) (width 0.2) (layer "F.Cu") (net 3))
 (segment (start 118 128) (end 117.65 128.35) (width 0.2) (layer "F.Cu") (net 3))
 (via (at 118 127) (size 0.6) (drill 0.3) (layers "F.Cu" "B.Cu") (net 3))
 (via (at 107.5 121) (size 0.6) (drill 0.3) (layers "F.Cu" "B.Cu") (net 3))
 (via (at 118 127) (size 0.6) (drill 0.3) (layers "F.Cu" "B.Cu") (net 3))
 (via (at 107.5 121) (size 0.6) (drill 0.3) (layers "F.Cu" "B.Cu") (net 3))
 (via (at 118 127) (size 0.6) (drill 0.3) (layers "F.Cu" "B.Cu") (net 3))
 (segment (start 117 126) (end 118 127) (width 0.2) (layer "B.Cu") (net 3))
 (segment (start 107.5 121) (end 108.5 121) (width 0.2) (layer "B.Cu") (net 3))
 (segment (start 108.5 121) (end 113.5 126) (width 0.2) (layer "B.Cu") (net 3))
 (segment (start 113.5 126) (end 117 126) (width 0.2) (layer "B.Cu") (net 3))
 (segment (start 123.75 133.25) (end 124 133) (width 0.2) (layer "F.Cu") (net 12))
 (segment (start 123.5925 133.25) (end 123.75 133.25) (width 0.2) (layer "F.Cu") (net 12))
 (segment (start 109.4025 136) (end 113.4025 140) (width 0.2) (layer "F.Cu") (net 12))
 (segment (start 120.25 133.25) (end 116 129) (width 0.2) (layer "F.Cu") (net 12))
 (segment (start 107.9875 135.9875) (end 107.5 135.5) (width 0.2) (layer "F.Cu") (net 12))
 (segment (start 115.5 138) (end 115.9025 138) (width 0.2) (layer "F.Cu") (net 12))
 (segment (start 123.5925 133.25) (end 120.25 133.25) (width 0.2) (layer "F.Cu") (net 12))
 (segment (start 113.5 138) (end 113.4025 138.0975) (width 0.2) (layer "F.Cu") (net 12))
 (segment (start 119.3425 137.5) (end 123.5925 133.25) (width 0.2) (layer "F.Cu") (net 12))
 (segment (start 116.4025 137.5) (end 119.3425 137.5) (width 0.2) (layer "F.Cu") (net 12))
 (segment (start 108 136) (end 109.4025 136) (width 0.2) (layer "F.Cu") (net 12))
 (segment (start 115.9025 138) (end 116.4025 137.5) (width 0.2) (layer "F.Cu") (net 12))
 (segment (start 113.4025 140) (end 113.4025 138.0975) (width 0.2) (layer "F.Cu") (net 12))
 (segment (start 107.9875 136.65) (end 107.9875 135.9875) (width 0.2) (layer "F.Cu") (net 12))
 (via (at 115.5 138) (size 0.6) (drill 0.3) (layers "F.Cu" "B.Cu") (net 12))
 (via (at 115.5 138) (size 0.6) (drill 0.3) (layers "F.Cu" "B.Cu") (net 12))
 (via (at 113.5 138) (size 0.6) (drill 0.3) (layers "F.Cu" "B.Cu") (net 12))
 (via (at 113.5 138) (size 0.6) (drill 0.3) (layers "F.Cu" "B.Cu") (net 12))
 (segment (start 113.5 138) (end 115.5 138) (width 0.2) (layer "B.Cu") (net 12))
 (segment (start 109 128.01) (end 109 125.352057) (width 0.2) (layer "F.Cu") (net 9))
 (segment (start 107.472943 123.825) (end 105.8875 123.825) (width 0.2) (layer "F.Cu") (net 9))
 (segment (start 109 125.352057) (end 107.472943 123.825) (width 0.2) (layer "F.Cu") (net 9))
 (segment (start 117.49 136.5) (end 109 128.01) (width 0.2) (layer "F.Cu") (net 9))
 (segment (start 108.5975 129.5) (end 109.5 129.5) (width 0.2) (layer "F.Cu") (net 11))
 (segment (start 111.675 123.825) (end 110.1125 123.825) (width 0.2) (layer "F.Cu") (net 11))
 (segment (start 112.5 123) (end 111.675 123.825) (width 0.2) (layer "F.Cu") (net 11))
 (segment (start 109.5 129.5) (end 110 130) (width 0.2) (layer "F.Cu") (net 11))
 (segment (start 108.5975 129.5) (end 108.5975 129.4025) (width 0.2) (layer "F.Cu") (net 11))
 (segment (start 113.5 127) (end 113.5 124) (width 0.2) (layer "F.Cu") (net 11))
 (via (at 112.5 123) (size 0.6) (drill 0.3) (layers "F.Cu" "B.Cu") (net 11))
 (via (at 110 130) (size 0.6) (drill 0.3) (layers "F.Cu" "B.Cu") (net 11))
 (via (at 110 130) (size 0.6) (drill 0.3) (layers "F.Cu" "B.Cu") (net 11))
 (via (at 112.5 123) (size 0.6) (drill 0.3) (layers "F.Cu" "B.Cu") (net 11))
 (via (at 113.5 124) (size 0.6) (drill 0.3) (layers "F.Cu" "B.Cu") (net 11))
 (via (at 110 130) (size 0.6) (drill 0.3) (layers "F.Cu" "B.Cu") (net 11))
 (via (at 113.5 127) (size 0.6) (drill 0.3) (layers "F.Cu" "B.Cu") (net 11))
 (via (at 113.5 127) (size 0.6) (drill 0.3) (layers "F.Cu" "B.Cu") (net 11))
 (segment (start 110 130.849943) (end 110.751057 131.601) (width 0.2) (layer "B.Cu") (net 11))
 (segment (start 113.5 129.349943) (end 113.5 127) (width 0.2) (layer "B.Cu") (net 11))
 (segment (start 111.248943 131.601) (end 113.5 129.349943) (width 0.2) (layer "B.Cu") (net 11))
 (segment (start 113.5 124) (end 112.5 123) (width 0.2) (layer "B.Cu") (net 11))
 (segment (start 110.751057 131.601) (end 111.248943 131.601) (width 0.2) (layer "B.Cu") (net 11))
 (segment (start 110 130) (end 110 130.849943) (width 0.2) (layer "B.Cu") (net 11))
 (segment (start 114.5975 140) (end 114.5975 134.5975) (width 0.2) (layer "F.Cu") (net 6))
 (segment (start 118 124) (end 116.5 122.5) (width 0.2) (layer "F.Cu") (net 6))
 (segment (start 110.5 127) (end 110.5 124.8625) (width 0.2) (layer "F.Cu") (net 6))
 (segment (start 112.025 124.475) (end 110.1125 124.475) (width 0.2) (layer "F.Cu") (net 6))
 (segment (start 114 122.5) (end 112.025 124.475) (width 0.2) (layer "F.Cu") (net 6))
 (segment (start 110.5 124.8625) (end 110.1125 124.475) (width 0.2) (layer "F.Cu") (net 6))
 (segment (start 116.5 122.5) (end 114 122.5) (width 0.2) (layer "F.Cu") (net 6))
 (segment (start 114.5975 134.5975) (end 111 131) (width 0.2) (layer "F.Cu") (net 6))
 (via (at 110.5 127) (size 0.6) (drill 0.3) (layers "F.Cu" "B.Cu") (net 6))
 (via (at 111 131) (size 0.6) (drill 0.3) (layers "F.Cu" "B.Cu") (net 6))
 (via (at 111 131) (size 0.6) (drill 0.3) (layers "F.Cu" "B.Cu") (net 6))
 (segment (start 111 131) (end 111 127.5) (width 0.2) (layer "B.Cu") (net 6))
 (segment (start 111 127.5) (end 110.5 127) (width 0.2) (layer "B.Cu") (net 6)))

